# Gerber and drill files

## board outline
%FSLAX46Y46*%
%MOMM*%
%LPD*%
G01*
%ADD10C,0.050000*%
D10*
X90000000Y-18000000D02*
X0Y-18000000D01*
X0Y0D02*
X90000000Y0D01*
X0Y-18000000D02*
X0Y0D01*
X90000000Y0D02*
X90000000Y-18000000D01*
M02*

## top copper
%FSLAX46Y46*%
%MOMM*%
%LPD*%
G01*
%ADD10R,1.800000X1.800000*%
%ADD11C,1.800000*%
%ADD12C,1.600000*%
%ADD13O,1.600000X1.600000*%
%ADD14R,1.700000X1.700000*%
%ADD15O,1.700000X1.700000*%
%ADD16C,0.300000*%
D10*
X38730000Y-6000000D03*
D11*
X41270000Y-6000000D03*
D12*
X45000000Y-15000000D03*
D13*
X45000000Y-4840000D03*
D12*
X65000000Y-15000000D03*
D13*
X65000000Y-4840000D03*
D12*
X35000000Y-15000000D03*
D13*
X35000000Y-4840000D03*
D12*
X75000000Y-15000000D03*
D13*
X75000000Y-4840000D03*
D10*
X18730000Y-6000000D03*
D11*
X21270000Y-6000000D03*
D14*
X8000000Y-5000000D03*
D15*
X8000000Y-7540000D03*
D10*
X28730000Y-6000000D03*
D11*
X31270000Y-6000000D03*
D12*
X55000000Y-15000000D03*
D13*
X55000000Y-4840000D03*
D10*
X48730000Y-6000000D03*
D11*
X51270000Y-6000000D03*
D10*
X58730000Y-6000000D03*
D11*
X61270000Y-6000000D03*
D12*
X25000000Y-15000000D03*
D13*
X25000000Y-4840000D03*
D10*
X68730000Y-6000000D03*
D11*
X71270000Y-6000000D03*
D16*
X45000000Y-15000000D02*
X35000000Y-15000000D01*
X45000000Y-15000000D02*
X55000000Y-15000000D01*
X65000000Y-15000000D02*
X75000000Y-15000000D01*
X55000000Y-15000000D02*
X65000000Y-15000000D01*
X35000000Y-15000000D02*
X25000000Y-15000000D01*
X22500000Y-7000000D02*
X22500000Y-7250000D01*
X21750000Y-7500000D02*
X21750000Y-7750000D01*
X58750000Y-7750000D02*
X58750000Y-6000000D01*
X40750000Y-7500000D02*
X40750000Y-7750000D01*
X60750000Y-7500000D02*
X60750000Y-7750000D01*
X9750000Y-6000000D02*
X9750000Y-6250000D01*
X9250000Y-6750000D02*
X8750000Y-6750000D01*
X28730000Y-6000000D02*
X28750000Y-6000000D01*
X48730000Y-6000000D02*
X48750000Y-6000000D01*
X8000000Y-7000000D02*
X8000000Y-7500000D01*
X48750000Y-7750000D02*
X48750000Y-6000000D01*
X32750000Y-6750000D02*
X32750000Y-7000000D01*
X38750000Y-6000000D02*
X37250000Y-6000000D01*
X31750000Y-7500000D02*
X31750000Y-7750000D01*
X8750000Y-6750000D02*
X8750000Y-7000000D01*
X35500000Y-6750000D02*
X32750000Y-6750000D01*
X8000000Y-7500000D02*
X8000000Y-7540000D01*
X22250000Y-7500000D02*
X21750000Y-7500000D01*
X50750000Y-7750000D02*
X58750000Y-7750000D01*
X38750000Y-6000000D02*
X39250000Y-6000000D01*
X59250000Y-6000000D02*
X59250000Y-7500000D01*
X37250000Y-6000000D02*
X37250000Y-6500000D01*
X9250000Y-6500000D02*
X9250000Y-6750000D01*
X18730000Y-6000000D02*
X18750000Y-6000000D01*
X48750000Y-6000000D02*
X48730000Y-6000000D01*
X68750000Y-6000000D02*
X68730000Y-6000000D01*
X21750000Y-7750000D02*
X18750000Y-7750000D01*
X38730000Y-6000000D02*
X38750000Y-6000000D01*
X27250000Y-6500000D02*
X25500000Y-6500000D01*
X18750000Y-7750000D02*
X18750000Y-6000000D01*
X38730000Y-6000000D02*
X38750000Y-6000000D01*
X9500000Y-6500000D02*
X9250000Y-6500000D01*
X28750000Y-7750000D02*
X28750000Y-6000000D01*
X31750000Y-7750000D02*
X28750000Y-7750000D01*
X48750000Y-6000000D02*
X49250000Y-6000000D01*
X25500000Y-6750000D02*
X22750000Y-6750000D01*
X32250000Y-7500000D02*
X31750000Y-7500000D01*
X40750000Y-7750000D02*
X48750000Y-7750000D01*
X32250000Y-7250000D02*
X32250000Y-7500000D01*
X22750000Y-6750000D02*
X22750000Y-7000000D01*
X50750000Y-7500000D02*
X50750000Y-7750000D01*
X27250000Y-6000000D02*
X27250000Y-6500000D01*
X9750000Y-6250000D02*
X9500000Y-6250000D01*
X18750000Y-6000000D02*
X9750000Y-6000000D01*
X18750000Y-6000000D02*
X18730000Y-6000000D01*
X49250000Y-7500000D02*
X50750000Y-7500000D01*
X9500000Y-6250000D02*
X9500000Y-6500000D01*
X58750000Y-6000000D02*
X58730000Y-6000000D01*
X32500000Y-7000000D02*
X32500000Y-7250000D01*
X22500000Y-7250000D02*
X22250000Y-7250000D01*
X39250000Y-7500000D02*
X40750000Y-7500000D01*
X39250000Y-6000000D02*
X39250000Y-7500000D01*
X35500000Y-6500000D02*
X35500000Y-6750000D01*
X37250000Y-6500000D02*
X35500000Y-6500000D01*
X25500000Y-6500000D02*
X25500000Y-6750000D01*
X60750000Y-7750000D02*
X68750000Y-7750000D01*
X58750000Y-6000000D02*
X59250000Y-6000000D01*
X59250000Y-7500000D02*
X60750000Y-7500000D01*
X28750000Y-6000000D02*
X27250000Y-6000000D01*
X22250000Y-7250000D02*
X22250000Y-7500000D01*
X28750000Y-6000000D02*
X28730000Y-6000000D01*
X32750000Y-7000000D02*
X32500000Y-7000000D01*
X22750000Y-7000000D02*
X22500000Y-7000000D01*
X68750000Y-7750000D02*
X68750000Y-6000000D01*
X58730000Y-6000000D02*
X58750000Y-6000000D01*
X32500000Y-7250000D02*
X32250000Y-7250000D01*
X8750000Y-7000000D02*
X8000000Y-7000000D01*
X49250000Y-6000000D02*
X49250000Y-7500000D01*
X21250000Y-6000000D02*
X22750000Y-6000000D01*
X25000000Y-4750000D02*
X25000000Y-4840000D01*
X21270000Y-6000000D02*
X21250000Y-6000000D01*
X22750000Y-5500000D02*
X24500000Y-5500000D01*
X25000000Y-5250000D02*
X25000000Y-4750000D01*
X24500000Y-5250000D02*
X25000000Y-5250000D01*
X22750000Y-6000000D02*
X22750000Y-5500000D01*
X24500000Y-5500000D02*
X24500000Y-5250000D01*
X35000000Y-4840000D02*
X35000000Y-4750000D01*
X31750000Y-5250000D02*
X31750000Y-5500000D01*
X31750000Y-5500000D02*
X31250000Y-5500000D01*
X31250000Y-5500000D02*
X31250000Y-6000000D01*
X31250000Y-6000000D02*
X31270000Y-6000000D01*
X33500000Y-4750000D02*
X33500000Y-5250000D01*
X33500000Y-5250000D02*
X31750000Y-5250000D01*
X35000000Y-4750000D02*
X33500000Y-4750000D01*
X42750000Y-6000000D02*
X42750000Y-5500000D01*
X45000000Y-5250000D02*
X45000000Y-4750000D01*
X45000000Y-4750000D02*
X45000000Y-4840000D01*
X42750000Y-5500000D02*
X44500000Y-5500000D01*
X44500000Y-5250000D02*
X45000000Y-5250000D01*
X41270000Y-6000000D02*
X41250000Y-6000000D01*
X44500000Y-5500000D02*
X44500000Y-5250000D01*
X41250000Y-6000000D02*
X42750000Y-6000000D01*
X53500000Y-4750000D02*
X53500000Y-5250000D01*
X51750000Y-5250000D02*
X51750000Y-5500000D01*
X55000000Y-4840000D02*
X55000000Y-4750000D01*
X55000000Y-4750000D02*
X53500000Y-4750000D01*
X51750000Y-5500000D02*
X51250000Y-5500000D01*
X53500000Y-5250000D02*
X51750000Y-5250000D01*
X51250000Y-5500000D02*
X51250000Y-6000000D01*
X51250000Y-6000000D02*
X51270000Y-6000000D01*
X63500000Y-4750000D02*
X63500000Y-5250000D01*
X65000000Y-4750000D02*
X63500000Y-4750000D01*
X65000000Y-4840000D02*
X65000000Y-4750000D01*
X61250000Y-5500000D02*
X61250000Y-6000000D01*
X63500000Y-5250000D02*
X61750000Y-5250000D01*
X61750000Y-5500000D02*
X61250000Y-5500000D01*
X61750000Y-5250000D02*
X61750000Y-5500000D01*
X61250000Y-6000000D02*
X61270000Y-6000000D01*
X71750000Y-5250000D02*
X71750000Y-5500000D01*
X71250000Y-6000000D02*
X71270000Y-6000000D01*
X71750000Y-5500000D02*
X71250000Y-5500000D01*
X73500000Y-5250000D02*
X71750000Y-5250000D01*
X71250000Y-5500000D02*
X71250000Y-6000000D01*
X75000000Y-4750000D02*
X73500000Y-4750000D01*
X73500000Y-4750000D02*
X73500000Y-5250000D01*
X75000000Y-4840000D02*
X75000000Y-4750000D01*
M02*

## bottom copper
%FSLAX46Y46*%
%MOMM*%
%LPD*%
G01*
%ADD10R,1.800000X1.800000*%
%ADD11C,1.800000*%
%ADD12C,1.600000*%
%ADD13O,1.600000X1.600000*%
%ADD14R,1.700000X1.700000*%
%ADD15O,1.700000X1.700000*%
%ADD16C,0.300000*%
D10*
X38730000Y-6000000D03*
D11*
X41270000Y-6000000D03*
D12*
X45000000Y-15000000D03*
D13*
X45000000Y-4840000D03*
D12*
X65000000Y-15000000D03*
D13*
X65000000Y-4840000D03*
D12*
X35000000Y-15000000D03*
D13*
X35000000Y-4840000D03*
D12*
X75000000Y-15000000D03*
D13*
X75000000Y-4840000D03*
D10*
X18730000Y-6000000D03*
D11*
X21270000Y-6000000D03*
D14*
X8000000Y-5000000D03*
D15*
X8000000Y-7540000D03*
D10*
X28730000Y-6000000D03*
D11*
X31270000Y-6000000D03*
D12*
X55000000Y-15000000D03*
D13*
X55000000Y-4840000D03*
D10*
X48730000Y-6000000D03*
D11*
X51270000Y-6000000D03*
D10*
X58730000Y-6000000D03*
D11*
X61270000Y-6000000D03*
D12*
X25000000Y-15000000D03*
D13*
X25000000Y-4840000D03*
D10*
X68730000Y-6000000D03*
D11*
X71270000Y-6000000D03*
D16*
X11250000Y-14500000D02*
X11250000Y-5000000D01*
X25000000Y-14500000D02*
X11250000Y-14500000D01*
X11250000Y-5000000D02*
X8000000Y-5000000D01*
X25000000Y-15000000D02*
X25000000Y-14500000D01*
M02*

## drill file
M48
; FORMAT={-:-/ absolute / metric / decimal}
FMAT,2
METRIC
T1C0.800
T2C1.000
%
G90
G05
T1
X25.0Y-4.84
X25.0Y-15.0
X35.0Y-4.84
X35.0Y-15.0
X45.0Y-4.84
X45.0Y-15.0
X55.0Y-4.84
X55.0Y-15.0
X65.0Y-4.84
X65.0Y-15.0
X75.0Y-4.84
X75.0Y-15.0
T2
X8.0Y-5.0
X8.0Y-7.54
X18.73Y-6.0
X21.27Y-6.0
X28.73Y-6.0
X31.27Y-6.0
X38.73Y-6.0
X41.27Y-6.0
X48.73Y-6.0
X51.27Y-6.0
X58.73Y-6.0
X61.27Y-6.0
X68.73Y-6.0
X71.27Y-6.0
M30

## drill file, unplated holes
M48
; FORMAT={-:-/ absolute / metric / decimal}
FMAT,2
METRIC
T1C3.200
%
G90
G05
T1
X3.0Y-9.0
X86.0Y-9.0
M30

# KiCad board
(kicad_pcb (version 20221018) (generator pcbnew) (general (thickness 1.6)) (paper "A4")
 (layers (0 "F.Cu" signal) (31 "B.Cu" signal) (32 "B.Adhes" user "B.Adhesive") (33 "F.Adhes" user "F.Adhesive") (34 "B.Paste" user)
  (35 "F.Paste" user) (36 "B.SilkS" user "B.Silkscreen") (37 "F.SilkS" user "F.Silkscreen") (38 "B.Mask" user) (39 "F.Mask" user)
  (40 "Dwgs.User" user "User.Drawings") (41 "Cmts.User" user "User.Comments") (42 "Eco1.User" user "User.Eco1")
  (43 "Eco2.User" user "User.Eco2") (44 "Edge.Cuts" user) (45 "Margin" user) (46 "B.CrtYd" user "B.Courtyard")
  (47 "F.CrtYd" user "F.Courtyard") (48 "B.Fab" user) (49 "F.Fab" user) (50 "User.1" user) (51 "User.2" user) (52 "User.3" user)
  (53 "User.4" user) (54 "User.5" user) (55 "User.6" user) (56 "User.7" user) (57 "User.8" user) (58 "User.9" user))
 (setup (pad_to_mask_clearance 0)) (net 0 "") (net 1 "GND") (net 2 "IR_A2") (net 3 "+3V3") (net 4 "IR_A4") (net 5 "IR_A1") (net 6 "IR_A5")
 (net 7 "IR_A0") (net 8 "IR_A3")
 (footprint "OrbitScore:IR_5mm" (layer "F.Cu") (at 40 6)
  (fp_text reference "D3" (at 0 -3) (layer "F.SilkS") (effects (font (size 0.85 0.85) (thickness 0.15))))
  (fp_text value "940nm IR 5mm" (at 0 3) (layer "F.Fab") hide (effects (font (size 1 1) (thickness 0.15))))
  (pad "1" thru_hole rect (at -1.27 0) (size 1.8 1.8) (drill 1) (layers "*.Cu" "*.Mask") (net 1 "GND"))
  (pad "2" thru_hole circle (at 1.27 0) (size 1.8 1.8) (drill 1) (layers "*.Cu" "*.Mask") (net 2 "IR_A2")))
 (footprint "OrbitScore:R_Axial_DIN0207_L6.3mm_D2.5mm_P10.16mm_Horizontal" (layer "F.Cu") (at 45 15 90)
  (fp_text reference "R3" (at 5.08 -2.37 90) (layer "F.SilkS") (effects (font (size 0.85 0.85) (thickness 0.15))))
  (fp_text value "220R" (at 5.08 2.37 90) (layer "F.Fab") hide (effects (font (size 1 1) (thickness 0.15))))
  (pad "1" thru_hole circle (at 0 0 90) (size 1.6 1.6) (drill 0.8) (layers "*.Cu" "*.Mask") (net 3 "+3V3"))
  (pad "2" thru_hole oval (at 10.16 0 90) (size 1.6 1.6) (drill 0.8) (layers "*.Cu" "*.Mask") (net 2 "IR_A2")))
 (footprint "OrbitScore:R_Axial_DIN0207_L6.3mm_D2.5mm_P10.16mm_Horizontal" (layer "F.Cu") (at 65 15 90)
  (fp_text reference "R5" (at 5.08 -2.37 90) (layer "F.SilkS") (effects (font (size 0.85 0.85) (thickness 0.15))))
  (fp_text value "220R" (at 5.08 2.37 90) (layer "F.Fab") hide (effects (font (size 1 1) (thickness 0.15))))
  (pad "1" thru_hole circle (at 0 0 90) (size 1.6 1.6) (drill 0.8) (layers "*.Cu" "*.Mask") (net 3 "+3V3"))
  (pad "2" thru_hole oval (at 10.16 0 90) (size 1.6 1.6) (drill 0.8) (layers "*.Cu" "*.Mask") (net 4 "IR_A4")))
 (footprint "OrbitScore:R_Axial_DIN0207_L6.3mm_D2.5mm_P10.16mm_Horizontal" (layer "F.Cu") (at 35 15 90)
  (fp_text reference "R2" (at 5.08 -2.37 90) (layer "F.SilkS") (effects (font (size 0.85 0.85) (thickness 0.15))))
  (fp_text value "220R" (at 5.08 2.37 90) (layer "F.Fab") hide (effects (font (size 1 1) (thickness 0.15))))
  (pad "1" thru_hole circle (at 0 0 90) (size 1.6 1.6) (drill 0.8) (layers "*.Cu" "*.Mask") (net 3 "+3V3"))
  (pad "2" thru_hole oval (at 10.16 0 90) (size 1.6 1.6) (drill 0.8) (layers "*.Cu" "*.Mask") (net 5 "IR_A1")))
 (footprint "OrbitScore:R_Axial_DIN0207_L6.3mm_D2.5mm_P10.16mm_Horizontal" (layer "F.Cu") (at 75 15 90)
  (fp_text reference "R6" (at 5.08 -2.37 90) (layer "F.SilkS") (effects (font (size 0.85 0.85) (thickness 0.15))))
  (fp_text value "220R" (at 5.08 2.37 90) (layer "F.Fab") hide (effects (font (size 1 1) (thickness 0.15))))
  (pad "1" thru_hole circle (at 0 0 90) (size 1.6 1.6) (drill 0.8) (layers "*.Cu" "*.Mask") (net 3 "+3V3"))
  (pad "2" thru_hole oval (at 10.16 0 90) (size 1.6 1.6) (drill 0.8) (layers "*.Cu" "*.Mask") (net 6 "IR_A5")))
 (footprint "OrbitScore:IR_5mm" (layer "F.Cu") (at 20 6)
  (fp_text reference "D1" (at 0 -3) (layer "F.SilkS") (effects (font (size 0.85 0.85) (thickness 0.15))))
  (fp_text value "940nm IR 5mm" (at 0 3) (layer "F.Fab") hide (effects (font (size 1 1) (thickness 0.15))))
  (pad "1" thru_hole rect (at -1.27 0) (size 1.8 1.8) (drill 1) (layers "*.Cu" "*.Mask") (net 1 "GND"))
  (pad "2" thru_hole circle (at 1.27 0) (size 1.8 1.8) (drill 1) (layers "*.Cu" "*.Mask") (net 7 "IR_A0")))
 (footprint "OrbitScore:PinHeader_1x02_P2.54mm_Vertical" (layer "F.Cu") (at 8 5)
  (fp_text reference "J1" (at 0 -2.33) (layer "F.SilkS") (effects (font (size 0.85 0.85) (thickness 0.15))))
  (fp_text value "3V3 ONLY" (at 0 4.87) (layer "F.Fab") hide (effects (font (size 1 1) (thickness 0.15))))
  (pad "1" thru_hole rect (at 0 0) (size 1.7 1.7) (drill 1) (layers "*.Cu" "*.Mask") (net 3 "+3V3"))
  (pad "2" thru_hole oval (at 0 2.54) (size 1.7 1.7) (drill 1) (layers "*.Cu" "*.Mask") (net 1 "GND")))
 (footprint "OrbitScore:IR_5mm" (layer "F.Cu") (at 30 6)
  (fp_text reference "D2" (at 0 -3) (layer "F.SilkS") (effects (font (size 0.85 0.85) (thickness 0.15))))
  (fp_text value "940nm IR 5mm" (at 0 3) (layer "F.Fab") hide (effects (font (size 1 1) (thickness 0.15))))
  (pad "1" thru_hole rect (at -1.27 0) (size 1.8 1.8) (drill 1) (layers "*.Cu" "*.Mask") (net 1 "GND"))
  (pad "2" thru_hole circle (at 1.27 0) (size 1.8 1.8) (drill 1) (layers "*.Cu" "*.Mask") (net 5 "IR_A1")))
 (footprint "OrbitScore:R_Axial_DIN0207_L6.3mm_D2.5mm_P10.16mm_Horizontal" (layer "F.Cu") (at 55 15 90)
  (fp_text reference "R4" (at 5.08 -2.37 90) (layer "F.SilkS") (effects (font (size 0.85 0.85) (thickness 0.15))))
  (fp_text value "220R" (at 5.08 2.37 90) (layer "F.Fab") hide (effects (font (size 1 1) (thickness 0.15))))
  (pad "1" thru_hole circle (at 0 0 90) (size 1.6 1.6) (drill 0.8) (layers "*.Cu" "*.Mask") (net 3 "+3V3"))
  (pad "2" thru_hole oval (at 10.16 0 90) (size 1.6 1.6) (drill 0.8) (layers "*.Cu" "*.Mask") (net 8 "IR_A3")))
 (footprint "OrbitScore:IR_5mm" (layer "F.Cu") (at 50 6)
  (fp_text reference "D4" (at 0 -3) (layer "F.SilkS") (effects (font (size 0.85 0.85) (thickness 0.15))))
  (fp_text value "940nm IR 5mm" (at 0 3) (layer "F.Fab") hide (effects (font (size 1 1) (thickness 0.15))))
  (pad "1" thru_hole rect (at -1.27 0) (size 1.8 1.8) (drill 1) (layers "*.Cu" "*.Mask") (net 1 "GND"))
  (pad "2" thru_hole circle (at 1.27 0) (size 1.8 1.8) (drill 1) (layers "*.Cu" "*.Mask") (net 8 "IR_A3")))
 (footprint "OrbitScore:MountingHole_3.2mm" (layer "F.Cu") (at 3 9)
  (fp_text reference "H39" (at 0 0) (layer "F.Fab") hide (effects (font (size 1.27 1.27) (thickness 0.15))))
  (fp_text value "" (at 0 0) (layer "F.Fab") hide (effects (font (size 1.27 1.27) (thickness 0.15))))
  (pad "" np_thru_hole circle (at 0 0) (size 3.2 3.2) (drill 3.2) (layers "*.Cu" "*.Mask")))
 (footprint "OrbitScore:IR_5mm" (layer "F.Cu") (at 60 6)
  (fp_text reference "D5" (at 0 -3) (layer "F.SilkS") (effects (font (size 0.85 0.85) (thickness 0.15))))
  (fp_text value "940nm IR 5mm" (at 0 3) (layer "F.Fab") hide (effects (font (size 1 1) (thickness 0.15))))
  (pad "1" thru_hole rect (at -1.27 0) (size 1.8 1.8) (drill 1) (layers "*.Cu" "*.Mask") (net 1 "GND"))
  (pad "2" thru_hole circle (at 1.27 0) (size 1.8 1.8) (drill 1) (layers "*.Cu" "*.Mask") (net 4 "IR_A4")))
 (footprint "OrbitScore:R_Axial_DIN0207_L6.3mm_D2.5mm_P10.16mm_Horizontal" (layer "F.Cu") (at 25 15 90)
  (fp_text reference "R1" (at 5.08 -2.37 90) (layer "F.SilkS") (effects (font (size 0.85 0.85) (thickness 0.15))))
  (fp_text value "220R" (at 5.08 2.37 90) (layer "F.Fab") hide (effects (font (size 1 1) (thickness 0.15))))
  (pad "1" thru_hole circle (at 0 0 90) (size 1.6 1.6) (drill 0.8) (layers "*.Cu" "*.Mask") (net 3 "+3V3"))
  (pad "2" thru_hole oval (at 10.16 0 90) (size 1.6 1.6) (drill 0.8) (layers "*.Cu" "*.Mask") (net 7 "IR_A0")))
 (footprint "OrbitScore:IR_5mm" (layer "F.Cu") (at 70 6)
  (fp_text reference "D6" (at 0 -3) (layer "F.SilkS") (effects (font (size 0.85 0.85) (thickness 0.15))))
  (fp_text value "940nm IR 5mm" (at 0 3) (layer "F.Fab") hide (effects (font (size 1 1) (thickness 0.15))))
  (pad "1" thru_hole rect (at -1.27 0) (size 1.8 1.8) (drill 1) (layers "*.Cu" "*.Mask") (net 1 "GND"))
  (pad "2" thru_hole circle (at 1.27 0) (size 1.8 1.8) (drill 1) (layers "*.Cu" "*.Mask") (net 6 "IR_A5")))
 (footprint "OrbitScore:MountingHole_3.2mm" (layer "F.Cu") (at 86 9)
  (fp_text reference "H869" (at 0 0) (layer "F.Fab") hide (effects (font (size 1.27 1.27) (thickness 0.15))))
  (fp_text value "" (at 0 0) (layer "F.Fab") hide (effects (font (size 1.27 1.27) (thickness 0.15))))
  (pad "" np_thru_hole circle (at 0 0) (size 3.2 3.2) (drill 3.2) (layers "*.Cu" "*.Mask")))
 (gr_line (start 90 18) (end 0 18) (stroke (width 0.05) (type default)) (layer "Edge.Cuts"))
 (gr_line (start 0 0) (end 90 0) (stroke (width 0.05) (type default)) (layer "Edge.Cuts"))
 (gr_line (start 0 18) (end 0 0) (stroke (width 0.05) (type default)) (layer "Edge.Cuts"))
 (gr_line (start 90 0) (end 90 18) (stroke (width 0.05) (type default)) (layer "Edge.Cuts"))
 (segment (start 45 15) (end 35 15) (width 0.3) (layer "F.Cu") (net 3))
 (segment (start 45 15) (end 55 15) (width 0.3) (layer "F.Cu") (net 3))
 (segment (start 65 15) (end 75 15) (width 0.3) (layer "F.Cu") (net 3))
 (segment (start 55 15) (end 65 15) (width 0.3) (layer "F.Cu") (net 3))
 (segment (start 35 15) (end 25 15) (width 0.3) (layer "F.Cu") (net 3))
 (segment (start 11.25 14.5) (end 11.25 5) (width 0.3) (layer "B.Cu") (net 3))
 (segment (start 25 14.5) (end 11.25 14.5) (width 0.3) (layer "B.Cu") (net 3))
 (segment (start 11.25 5) (end 8 5) (width 0.3) (layer "B.Cu") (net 3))
 (segment (start 25 15) (end 25 14.5) (width 0.3) (layer "B.Cu") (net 3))
 (segment (start 22.5 7) (end 22.5 7.25) (width 0.3) (layer "F.Cu") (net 1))
 (segment (start 21.75 7.5) (end 21.75 7.75) (width 0.3) (layer "F.Cu") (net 1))
 (segment (start 58.75 7.75) (end 58.75 6) (width 0.3) (layer "F.Cu") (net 1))
 (segment (start 40.75 7.5) (end 40.75 7.75) (width 0.3) (layer "F.Cu") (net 1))
 (segment (start 60.75 7.5) (end 60.75 7.75) (width 0.3) (layer "F.Cu") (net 1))
 (segment (start 9.75 6) (end 9.75 6.25) (width 0.3) (layer "F.Cu") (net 1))
 (segment (start 9.25 6.75) (end 8.75 6.75) (width 0.3) (layer "F.Cu") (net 1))
 (segment (start 28.73 6) (end 28.75 6) (width 0.3) (layer "F.Cu") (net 1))
 (segment (start 48.73 6) (end 48.75 6) (width 0.3) (layer "F.Cu") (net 1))
 (segment (start 8 7) (end 8 7.5) (width 0.3) (layer "F.Cu") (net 1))
 (segment (start 48.75 7.75) (end 48.75 6) (width 0.3) (layer "F.Cu") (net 1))
 (segment (start 32.75 6.75) (end 32.75 7) (width 0.3) (layer "F.Cu") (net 1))
 (segment (start 38.75 6) (end 37.25 6) (width 0.3) (layer "F.Cu") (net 1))
 (segment (start 31.75 7.5) (end 31.75 7.75) (width 0.3) (layer "F.Cu") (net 1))
 (segment (start 8.75 6.75) (end 8.75 7) (width 0.3) (layer "F.Cu") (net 1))
 (segment (start 35.5 6.75) (end 32.75 6.75) (width 0.3) (layer "F.Cu") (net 1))
 (segment (start 8 7.5) (end 8 7.54) (width 0.3) (layer "F.Cu") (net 1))
 (segment (start 22.25 7.5) (end 21.75 7.5) (width 0.3) (layer "F.Cu") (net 1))
 (segment (start 50.75 7.75) (end 58.75 7.75) (width 0.3) (layer "F.Cu") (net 1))
 (segment (start 38.75 6) (end 39.25 6) (width 0.3) (layer "F.Cu") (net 1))
 (segment (start 59.25 6) (end 59.25 7.5) (width 0.3) (layer "F.Cu") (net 1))
 (segment (start 37.25 6) (end 37.25 6.5) (width 0.3) (layer "F.Cu") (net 1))
 (segment (start 9.25 6.5) (end 9.25 6.75) (width 0.3) (layer "F.Cu") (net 1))
 (segment (start 18.73 6) (end 18.75 6) (width 0.3) (layer "F.Cu") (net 1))
 (segment (start 48.75 6) (end 48.73 6) (width 0.3) (layer "F.Cu") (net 1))
 (segment (start 68.75 6) (end 68.73 6) (width 0.3) (layer "F.Cu") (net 1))
 (segment (start 21.75 7.75) (end 18.75 7.75) (width 0.3) (layer "F.Cu") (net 1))
 (segment (start 38.73 6) (end 38.75 6) (width 0.3) (layer "F.Cu") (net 1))
 (segment (start 27.25 6.5) (end 25.5 6.5) (width 0.3) (layer "F.Cu") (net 1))
 (segment (start 18.75 7.75) (end 18.75 6) (width 0.3) (layer "F.Cu") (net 1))
 (segment (start 38.73 6) (end 38.75 6) (width 0.3) (layer "F.Cu") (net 1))
 (segment (start 9.5 6.5) (end 9.25 6.5) (width 0.3) (layer "F.Cu") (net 1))
 (segment (start 28.75 7.75) (end 28.75 6) (width 0.3) (layer "F.Cu") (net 1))
 (segment (start 31.75 7.75) (end 28.75 7.75) (width 0.3) (layer "F.Cu") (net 1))
 (segment (start 48.75 6) (end 49.25 6) (width 0.3) (layer "F.Cu") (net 1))
 (segment (start 25.5 6.75) (end 22.75 6.75) (width 0.3) (layer "F.Cu") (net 1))
 (segment (start 32.25 7.5) (end 31.75 7.5) (width 0.3) (layer "F.Cu") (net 1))
 (segment (start 40.75 7.75) (end 48.75 7.75) (width 0.3) (layer "F.Cu") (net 1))
 (segment (start 32.25 7.25) (end 32.25 7.5) (width 0.3) (layer "F.Cu") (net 1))
 (segment (start 22.75 6.75) (end 22.75 7) (width 0.3) (layer "F.Cu") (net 1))
 (segment (start 50.75 7.5) (end 50.75 7.75) (width 0.3) (layer "F.Cu") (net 1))
 (segment (start 27.25 6) (end 27.25 6.5) (width 0.3) (layer "F.Cu") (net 1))
 (segment (start 9.75 6.25) (end 9.5 6.25) (width 0.3) (layer "F.Cu") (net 1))
 (segment (start 18.75 6) (end 9.75 6) (width 0.3) (layer "F.Cu") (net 1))
 (segment (start 18.75 6) (end 18.73 6) (width 0.3) (layer "F.Cu") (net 1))
 (segment (start 49.25 7.5) (end 50.75 7.5) (width 0.3) (layer "F.Cu") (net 1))
 (segment (start 9.5 6.25) (end 9.5 6.5) (width 0.3) (layer "F.Cu") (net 1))
 (segment (start 58.75 6) (end 58.73 6) (width 0.3) (layer "F.Cu") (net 1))
 (segment (start 32.5 7) (end 32.5 7.25) (width 0.3) (layer "F.Cu") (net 1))
 (segment (start 22.5 7.25) (end 22.25 7.25) (width 0.3) (layer "F.Cu") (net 1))
 (segment (start 39.25 7.5) (end 40.75 7.5) (width 0.3) (layer "F.Cu") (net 1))
 (segment (start 39.25 6) (end 39.25 7.5) (width 0.3) (layer "F.Cu") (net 1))
 (segment (start 35.5 6.5) (end 35.5 6.75) (width 0.3) (layer "F.Cu") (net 1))
 (segment (start 37.25 6.5) (end 35.5 6.5) (width 0.3) (layer "F.Cu") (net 1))
 (segment (start 25.5 6.5) (end 25.5 6.75) (width 0.3) (layer "F.Cu") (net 1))
 (segment (start 60.75 7.75) (end 68.75 7.75) (width 0.3) (layer "F.Cu") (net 1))
 (segment (start 58.75 6) (end 59.25 6) (width 0.3) (layer "F.Cu") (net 1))
 (segment (start 59.25 7.5) (end 60.75 7.5) (width 0.3) (layer "F.Cu") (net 1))
 (segment (start 28.75 6) (end 27.25 6) (width 0.3) (layer "F.Cu") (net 1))
 (segment (start 22.25 7.25) (end 22.25 7.5) (width 0.3) (layer "F.Cu") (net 1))
 (segment (start 28.75 6) (end 28.73 6) (width 0.3) (layer "F.Cu") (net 1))
 (segment (start 32.75 7) (end 32.5 7) (width 0.3) (layer "F.Cu") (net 1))
 (segment (start 22.75 7) (end 22.5 7) (width 0.3) (layer "F.Cu") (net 1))
 (segment (start 68.75 7.75) (end 68.75 6) (width 0.3) (layer "F.Cu") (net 1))
 (segment (start 58.73 6) (end 58.75 6) (width 0.3) (layer "F.Cu") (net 1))
 (segment (start 32.5 7.25) (end 32.25 7.25) (width 0.3) (layer "F.Cu") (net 1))
 (segment (start 8.75 7) (end 8 7) (width 0.3) (layer "F.Cu") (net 1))
 (segment (start 49.25 6) (end 49.25 7.5) (width 0.3) (layer "F.Cu") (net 1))
 (segment (start 21.25 6) (end 22.75 6) (width 0.3) (layer "F.Cu") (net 7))
 (segment (start 25 4.75) (end 25 4.84) (width 0.3) (layer "F.Cu") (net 7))
 (segment (start 21.27 6) (end 21.25 6) (width 0.3) (layer "F.Cu") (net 7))
 (segment (start 22.75 5.5) (end 24.5 5.5) (width 0.3) (layer "F.Cu") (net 7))
 (segment (start 25 5.25) (end 25 4.75) (width 0.3) (layer "F.Cu") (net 7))
 (segment (start 24.5 5.25) (end 25 5.25) (width 0.3) (layer "F.Cu") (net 7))
 (segment (start 22.75 6) (end 22.75 5.5) (width 0.3) (layer "F.Cu") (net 7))
 (segment (start 24.5 5.5) (end 24.5 5.25) (width 0.3) (layer "F.Cu") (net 7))
 (segment (start 35 4.84) (end 35 4.75) (width 0.3) (layer "F.Cu") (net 5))
 (segment (start 31.75 5.25) (end 31.75 5.5) (width 0.3) (layer "F.Cu") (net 5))
 (segment (start 31.75 5.5) (end 31.25 5.5) (width 0.3) (layer "F.Cu") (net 5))
 (segment (start 31.25 5.5) (end 31.25 6) (width 0.3) (layer "F.Cu") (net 5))
 (segment (start 31.25 6) (end 31.27 6) (width 0.3) (layer "F.Cu") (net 5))
 (segment (start 33.5 4.75) (end 33.5 5.25) (width 0.3) (layer "F.Cu") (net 5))
 (segment (start 33.5 5.25) (end 31.75 5.25) (width 0.3) (layer "F.Cu") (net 5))
 (segment (start 35 4.75) (end 33.5 4.75) (width 0.3) (layer "F.Cu") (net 5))
 (segment (start 42.75 6) (end 42.75 5.5) (width 0.3) (layer "F.Cu") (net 2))
 (segment (start 45 5.25) (end 45 4.75) (width 0.3) (layer "F.Cu") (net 2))
 (segment (start 45 4.75) (end 45 4.84) (width 0.3) (layer "F.Cu") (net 2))
 (segment (start 42.75 5.5) (end 44.5 5.5) (width 0.3) (layer "F.Cu") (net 2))
 (segment (start 44.5 5.25) (end 45 5.25) (width 0.3) (layer "F.Cu") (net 2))
 (segment (start 41.27 6) (end 41.25 6) (width 0.3) (layer "F.Cu") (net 2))
 (segment (start 44.5 5.5) (end 44.5 5.25) (width 0.3) (layer "F.Cu") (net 2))
 (segment (start 41.25 6) (end 42.75 6) (width 0.3) (layer "F.Cu") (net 2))
 (segment (start 53.5 4.75) (end 53.5 5.25) (width 0.3) (layer "F.Cu") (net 8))
 (segment (start 51.75 5.25) (end 51.75 5.5) (width 0.3) (layer "F.Cu") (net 8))
 (segment (start 55 4.84) (end 55 4.75) (width 0.3) (layer "F.Cu") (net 8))
 (segment (start 55 4.75) (end 53.5 4.75) (width 0.3) (layer "F.Cu") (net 8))
 (segment (start 51.75 5.5) (end 51.25 5.5) (width 0.3) (layer "F.Cu") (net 8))
 (segment (start 53.5 5.25) (end 51.75 5.25) (width 0.3) (layer "F.Cu") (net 8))
 (segment (start 51.25 5.5) (end 51.25 6) (width 0.3) (layer "F.Cu") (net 8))
 (segment (start 51.25 6) (end 51.27 6) (width 0.3) (layer "F.Cu") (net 8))
 (segment (start 63.5 4.75) (end 63.5 5.25) (width 0.3) (layer "F.Cu") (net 4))
 (segment (start 65 4.75) (end 63.5 4.75) (width 0.3) (layer "F.Cu") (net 4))
 (segment (start 65 4.84) (end 65 4.75) (width 0.3) (layer "F.Cu") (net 4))
 (segment (start 61.25 5.5) (end 61.25 6) (width 0.3) (layer "F.Cu") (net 4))
 (segment (start 63.5 5.25) (end 61.75 5.25) (width 0.3) (layer "F.Cu") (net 4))
 (segment (start 61.75 5.5) (end 61.25 5.5) (width 0.3) (layer "F.Cu") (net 4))
 (segment (start 61.75 5.25) (end 61.75 5.5) (width 0.3) (layer "F.Cu") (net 4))
 (segment (start 61.25 6) (end 61.27 6) (width 0.3) (layer "F.Cu") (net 4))
 (segment (start 71.75 5.25) (end 71.75 5.5) (width 0.3) (layer "F.Cu") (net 6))
 (segment (start 71.25 6) (end 71.27 6) (width 0.3) (layer "F.Cu") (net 6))
 (segment (start 71.75 5.5) (end 71.25 5.5) (width 0.3) (layer "F.Cu") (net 6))
 (segment (start 73.5 5.25) (end 71.75 5.25) (width 0.3) (layer "F.Cu") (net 6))
 (segment (start 71.25 5.5) (end 71.25 6) (width 0.3) (layer "F.Cu") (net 6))
 (segment (start 75 4.75) (end 73.5 4.75) (width 0.3) (layer "F.Cu") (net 6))
 (segment (start 73.5 4.75) (end 73.5 5.25) (width 0.3) (layer "F.Cu") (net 6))
 (segment (start 75 4.84) (end 75 4.75) (width 0.3) (layer "F.Cu") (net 6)))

